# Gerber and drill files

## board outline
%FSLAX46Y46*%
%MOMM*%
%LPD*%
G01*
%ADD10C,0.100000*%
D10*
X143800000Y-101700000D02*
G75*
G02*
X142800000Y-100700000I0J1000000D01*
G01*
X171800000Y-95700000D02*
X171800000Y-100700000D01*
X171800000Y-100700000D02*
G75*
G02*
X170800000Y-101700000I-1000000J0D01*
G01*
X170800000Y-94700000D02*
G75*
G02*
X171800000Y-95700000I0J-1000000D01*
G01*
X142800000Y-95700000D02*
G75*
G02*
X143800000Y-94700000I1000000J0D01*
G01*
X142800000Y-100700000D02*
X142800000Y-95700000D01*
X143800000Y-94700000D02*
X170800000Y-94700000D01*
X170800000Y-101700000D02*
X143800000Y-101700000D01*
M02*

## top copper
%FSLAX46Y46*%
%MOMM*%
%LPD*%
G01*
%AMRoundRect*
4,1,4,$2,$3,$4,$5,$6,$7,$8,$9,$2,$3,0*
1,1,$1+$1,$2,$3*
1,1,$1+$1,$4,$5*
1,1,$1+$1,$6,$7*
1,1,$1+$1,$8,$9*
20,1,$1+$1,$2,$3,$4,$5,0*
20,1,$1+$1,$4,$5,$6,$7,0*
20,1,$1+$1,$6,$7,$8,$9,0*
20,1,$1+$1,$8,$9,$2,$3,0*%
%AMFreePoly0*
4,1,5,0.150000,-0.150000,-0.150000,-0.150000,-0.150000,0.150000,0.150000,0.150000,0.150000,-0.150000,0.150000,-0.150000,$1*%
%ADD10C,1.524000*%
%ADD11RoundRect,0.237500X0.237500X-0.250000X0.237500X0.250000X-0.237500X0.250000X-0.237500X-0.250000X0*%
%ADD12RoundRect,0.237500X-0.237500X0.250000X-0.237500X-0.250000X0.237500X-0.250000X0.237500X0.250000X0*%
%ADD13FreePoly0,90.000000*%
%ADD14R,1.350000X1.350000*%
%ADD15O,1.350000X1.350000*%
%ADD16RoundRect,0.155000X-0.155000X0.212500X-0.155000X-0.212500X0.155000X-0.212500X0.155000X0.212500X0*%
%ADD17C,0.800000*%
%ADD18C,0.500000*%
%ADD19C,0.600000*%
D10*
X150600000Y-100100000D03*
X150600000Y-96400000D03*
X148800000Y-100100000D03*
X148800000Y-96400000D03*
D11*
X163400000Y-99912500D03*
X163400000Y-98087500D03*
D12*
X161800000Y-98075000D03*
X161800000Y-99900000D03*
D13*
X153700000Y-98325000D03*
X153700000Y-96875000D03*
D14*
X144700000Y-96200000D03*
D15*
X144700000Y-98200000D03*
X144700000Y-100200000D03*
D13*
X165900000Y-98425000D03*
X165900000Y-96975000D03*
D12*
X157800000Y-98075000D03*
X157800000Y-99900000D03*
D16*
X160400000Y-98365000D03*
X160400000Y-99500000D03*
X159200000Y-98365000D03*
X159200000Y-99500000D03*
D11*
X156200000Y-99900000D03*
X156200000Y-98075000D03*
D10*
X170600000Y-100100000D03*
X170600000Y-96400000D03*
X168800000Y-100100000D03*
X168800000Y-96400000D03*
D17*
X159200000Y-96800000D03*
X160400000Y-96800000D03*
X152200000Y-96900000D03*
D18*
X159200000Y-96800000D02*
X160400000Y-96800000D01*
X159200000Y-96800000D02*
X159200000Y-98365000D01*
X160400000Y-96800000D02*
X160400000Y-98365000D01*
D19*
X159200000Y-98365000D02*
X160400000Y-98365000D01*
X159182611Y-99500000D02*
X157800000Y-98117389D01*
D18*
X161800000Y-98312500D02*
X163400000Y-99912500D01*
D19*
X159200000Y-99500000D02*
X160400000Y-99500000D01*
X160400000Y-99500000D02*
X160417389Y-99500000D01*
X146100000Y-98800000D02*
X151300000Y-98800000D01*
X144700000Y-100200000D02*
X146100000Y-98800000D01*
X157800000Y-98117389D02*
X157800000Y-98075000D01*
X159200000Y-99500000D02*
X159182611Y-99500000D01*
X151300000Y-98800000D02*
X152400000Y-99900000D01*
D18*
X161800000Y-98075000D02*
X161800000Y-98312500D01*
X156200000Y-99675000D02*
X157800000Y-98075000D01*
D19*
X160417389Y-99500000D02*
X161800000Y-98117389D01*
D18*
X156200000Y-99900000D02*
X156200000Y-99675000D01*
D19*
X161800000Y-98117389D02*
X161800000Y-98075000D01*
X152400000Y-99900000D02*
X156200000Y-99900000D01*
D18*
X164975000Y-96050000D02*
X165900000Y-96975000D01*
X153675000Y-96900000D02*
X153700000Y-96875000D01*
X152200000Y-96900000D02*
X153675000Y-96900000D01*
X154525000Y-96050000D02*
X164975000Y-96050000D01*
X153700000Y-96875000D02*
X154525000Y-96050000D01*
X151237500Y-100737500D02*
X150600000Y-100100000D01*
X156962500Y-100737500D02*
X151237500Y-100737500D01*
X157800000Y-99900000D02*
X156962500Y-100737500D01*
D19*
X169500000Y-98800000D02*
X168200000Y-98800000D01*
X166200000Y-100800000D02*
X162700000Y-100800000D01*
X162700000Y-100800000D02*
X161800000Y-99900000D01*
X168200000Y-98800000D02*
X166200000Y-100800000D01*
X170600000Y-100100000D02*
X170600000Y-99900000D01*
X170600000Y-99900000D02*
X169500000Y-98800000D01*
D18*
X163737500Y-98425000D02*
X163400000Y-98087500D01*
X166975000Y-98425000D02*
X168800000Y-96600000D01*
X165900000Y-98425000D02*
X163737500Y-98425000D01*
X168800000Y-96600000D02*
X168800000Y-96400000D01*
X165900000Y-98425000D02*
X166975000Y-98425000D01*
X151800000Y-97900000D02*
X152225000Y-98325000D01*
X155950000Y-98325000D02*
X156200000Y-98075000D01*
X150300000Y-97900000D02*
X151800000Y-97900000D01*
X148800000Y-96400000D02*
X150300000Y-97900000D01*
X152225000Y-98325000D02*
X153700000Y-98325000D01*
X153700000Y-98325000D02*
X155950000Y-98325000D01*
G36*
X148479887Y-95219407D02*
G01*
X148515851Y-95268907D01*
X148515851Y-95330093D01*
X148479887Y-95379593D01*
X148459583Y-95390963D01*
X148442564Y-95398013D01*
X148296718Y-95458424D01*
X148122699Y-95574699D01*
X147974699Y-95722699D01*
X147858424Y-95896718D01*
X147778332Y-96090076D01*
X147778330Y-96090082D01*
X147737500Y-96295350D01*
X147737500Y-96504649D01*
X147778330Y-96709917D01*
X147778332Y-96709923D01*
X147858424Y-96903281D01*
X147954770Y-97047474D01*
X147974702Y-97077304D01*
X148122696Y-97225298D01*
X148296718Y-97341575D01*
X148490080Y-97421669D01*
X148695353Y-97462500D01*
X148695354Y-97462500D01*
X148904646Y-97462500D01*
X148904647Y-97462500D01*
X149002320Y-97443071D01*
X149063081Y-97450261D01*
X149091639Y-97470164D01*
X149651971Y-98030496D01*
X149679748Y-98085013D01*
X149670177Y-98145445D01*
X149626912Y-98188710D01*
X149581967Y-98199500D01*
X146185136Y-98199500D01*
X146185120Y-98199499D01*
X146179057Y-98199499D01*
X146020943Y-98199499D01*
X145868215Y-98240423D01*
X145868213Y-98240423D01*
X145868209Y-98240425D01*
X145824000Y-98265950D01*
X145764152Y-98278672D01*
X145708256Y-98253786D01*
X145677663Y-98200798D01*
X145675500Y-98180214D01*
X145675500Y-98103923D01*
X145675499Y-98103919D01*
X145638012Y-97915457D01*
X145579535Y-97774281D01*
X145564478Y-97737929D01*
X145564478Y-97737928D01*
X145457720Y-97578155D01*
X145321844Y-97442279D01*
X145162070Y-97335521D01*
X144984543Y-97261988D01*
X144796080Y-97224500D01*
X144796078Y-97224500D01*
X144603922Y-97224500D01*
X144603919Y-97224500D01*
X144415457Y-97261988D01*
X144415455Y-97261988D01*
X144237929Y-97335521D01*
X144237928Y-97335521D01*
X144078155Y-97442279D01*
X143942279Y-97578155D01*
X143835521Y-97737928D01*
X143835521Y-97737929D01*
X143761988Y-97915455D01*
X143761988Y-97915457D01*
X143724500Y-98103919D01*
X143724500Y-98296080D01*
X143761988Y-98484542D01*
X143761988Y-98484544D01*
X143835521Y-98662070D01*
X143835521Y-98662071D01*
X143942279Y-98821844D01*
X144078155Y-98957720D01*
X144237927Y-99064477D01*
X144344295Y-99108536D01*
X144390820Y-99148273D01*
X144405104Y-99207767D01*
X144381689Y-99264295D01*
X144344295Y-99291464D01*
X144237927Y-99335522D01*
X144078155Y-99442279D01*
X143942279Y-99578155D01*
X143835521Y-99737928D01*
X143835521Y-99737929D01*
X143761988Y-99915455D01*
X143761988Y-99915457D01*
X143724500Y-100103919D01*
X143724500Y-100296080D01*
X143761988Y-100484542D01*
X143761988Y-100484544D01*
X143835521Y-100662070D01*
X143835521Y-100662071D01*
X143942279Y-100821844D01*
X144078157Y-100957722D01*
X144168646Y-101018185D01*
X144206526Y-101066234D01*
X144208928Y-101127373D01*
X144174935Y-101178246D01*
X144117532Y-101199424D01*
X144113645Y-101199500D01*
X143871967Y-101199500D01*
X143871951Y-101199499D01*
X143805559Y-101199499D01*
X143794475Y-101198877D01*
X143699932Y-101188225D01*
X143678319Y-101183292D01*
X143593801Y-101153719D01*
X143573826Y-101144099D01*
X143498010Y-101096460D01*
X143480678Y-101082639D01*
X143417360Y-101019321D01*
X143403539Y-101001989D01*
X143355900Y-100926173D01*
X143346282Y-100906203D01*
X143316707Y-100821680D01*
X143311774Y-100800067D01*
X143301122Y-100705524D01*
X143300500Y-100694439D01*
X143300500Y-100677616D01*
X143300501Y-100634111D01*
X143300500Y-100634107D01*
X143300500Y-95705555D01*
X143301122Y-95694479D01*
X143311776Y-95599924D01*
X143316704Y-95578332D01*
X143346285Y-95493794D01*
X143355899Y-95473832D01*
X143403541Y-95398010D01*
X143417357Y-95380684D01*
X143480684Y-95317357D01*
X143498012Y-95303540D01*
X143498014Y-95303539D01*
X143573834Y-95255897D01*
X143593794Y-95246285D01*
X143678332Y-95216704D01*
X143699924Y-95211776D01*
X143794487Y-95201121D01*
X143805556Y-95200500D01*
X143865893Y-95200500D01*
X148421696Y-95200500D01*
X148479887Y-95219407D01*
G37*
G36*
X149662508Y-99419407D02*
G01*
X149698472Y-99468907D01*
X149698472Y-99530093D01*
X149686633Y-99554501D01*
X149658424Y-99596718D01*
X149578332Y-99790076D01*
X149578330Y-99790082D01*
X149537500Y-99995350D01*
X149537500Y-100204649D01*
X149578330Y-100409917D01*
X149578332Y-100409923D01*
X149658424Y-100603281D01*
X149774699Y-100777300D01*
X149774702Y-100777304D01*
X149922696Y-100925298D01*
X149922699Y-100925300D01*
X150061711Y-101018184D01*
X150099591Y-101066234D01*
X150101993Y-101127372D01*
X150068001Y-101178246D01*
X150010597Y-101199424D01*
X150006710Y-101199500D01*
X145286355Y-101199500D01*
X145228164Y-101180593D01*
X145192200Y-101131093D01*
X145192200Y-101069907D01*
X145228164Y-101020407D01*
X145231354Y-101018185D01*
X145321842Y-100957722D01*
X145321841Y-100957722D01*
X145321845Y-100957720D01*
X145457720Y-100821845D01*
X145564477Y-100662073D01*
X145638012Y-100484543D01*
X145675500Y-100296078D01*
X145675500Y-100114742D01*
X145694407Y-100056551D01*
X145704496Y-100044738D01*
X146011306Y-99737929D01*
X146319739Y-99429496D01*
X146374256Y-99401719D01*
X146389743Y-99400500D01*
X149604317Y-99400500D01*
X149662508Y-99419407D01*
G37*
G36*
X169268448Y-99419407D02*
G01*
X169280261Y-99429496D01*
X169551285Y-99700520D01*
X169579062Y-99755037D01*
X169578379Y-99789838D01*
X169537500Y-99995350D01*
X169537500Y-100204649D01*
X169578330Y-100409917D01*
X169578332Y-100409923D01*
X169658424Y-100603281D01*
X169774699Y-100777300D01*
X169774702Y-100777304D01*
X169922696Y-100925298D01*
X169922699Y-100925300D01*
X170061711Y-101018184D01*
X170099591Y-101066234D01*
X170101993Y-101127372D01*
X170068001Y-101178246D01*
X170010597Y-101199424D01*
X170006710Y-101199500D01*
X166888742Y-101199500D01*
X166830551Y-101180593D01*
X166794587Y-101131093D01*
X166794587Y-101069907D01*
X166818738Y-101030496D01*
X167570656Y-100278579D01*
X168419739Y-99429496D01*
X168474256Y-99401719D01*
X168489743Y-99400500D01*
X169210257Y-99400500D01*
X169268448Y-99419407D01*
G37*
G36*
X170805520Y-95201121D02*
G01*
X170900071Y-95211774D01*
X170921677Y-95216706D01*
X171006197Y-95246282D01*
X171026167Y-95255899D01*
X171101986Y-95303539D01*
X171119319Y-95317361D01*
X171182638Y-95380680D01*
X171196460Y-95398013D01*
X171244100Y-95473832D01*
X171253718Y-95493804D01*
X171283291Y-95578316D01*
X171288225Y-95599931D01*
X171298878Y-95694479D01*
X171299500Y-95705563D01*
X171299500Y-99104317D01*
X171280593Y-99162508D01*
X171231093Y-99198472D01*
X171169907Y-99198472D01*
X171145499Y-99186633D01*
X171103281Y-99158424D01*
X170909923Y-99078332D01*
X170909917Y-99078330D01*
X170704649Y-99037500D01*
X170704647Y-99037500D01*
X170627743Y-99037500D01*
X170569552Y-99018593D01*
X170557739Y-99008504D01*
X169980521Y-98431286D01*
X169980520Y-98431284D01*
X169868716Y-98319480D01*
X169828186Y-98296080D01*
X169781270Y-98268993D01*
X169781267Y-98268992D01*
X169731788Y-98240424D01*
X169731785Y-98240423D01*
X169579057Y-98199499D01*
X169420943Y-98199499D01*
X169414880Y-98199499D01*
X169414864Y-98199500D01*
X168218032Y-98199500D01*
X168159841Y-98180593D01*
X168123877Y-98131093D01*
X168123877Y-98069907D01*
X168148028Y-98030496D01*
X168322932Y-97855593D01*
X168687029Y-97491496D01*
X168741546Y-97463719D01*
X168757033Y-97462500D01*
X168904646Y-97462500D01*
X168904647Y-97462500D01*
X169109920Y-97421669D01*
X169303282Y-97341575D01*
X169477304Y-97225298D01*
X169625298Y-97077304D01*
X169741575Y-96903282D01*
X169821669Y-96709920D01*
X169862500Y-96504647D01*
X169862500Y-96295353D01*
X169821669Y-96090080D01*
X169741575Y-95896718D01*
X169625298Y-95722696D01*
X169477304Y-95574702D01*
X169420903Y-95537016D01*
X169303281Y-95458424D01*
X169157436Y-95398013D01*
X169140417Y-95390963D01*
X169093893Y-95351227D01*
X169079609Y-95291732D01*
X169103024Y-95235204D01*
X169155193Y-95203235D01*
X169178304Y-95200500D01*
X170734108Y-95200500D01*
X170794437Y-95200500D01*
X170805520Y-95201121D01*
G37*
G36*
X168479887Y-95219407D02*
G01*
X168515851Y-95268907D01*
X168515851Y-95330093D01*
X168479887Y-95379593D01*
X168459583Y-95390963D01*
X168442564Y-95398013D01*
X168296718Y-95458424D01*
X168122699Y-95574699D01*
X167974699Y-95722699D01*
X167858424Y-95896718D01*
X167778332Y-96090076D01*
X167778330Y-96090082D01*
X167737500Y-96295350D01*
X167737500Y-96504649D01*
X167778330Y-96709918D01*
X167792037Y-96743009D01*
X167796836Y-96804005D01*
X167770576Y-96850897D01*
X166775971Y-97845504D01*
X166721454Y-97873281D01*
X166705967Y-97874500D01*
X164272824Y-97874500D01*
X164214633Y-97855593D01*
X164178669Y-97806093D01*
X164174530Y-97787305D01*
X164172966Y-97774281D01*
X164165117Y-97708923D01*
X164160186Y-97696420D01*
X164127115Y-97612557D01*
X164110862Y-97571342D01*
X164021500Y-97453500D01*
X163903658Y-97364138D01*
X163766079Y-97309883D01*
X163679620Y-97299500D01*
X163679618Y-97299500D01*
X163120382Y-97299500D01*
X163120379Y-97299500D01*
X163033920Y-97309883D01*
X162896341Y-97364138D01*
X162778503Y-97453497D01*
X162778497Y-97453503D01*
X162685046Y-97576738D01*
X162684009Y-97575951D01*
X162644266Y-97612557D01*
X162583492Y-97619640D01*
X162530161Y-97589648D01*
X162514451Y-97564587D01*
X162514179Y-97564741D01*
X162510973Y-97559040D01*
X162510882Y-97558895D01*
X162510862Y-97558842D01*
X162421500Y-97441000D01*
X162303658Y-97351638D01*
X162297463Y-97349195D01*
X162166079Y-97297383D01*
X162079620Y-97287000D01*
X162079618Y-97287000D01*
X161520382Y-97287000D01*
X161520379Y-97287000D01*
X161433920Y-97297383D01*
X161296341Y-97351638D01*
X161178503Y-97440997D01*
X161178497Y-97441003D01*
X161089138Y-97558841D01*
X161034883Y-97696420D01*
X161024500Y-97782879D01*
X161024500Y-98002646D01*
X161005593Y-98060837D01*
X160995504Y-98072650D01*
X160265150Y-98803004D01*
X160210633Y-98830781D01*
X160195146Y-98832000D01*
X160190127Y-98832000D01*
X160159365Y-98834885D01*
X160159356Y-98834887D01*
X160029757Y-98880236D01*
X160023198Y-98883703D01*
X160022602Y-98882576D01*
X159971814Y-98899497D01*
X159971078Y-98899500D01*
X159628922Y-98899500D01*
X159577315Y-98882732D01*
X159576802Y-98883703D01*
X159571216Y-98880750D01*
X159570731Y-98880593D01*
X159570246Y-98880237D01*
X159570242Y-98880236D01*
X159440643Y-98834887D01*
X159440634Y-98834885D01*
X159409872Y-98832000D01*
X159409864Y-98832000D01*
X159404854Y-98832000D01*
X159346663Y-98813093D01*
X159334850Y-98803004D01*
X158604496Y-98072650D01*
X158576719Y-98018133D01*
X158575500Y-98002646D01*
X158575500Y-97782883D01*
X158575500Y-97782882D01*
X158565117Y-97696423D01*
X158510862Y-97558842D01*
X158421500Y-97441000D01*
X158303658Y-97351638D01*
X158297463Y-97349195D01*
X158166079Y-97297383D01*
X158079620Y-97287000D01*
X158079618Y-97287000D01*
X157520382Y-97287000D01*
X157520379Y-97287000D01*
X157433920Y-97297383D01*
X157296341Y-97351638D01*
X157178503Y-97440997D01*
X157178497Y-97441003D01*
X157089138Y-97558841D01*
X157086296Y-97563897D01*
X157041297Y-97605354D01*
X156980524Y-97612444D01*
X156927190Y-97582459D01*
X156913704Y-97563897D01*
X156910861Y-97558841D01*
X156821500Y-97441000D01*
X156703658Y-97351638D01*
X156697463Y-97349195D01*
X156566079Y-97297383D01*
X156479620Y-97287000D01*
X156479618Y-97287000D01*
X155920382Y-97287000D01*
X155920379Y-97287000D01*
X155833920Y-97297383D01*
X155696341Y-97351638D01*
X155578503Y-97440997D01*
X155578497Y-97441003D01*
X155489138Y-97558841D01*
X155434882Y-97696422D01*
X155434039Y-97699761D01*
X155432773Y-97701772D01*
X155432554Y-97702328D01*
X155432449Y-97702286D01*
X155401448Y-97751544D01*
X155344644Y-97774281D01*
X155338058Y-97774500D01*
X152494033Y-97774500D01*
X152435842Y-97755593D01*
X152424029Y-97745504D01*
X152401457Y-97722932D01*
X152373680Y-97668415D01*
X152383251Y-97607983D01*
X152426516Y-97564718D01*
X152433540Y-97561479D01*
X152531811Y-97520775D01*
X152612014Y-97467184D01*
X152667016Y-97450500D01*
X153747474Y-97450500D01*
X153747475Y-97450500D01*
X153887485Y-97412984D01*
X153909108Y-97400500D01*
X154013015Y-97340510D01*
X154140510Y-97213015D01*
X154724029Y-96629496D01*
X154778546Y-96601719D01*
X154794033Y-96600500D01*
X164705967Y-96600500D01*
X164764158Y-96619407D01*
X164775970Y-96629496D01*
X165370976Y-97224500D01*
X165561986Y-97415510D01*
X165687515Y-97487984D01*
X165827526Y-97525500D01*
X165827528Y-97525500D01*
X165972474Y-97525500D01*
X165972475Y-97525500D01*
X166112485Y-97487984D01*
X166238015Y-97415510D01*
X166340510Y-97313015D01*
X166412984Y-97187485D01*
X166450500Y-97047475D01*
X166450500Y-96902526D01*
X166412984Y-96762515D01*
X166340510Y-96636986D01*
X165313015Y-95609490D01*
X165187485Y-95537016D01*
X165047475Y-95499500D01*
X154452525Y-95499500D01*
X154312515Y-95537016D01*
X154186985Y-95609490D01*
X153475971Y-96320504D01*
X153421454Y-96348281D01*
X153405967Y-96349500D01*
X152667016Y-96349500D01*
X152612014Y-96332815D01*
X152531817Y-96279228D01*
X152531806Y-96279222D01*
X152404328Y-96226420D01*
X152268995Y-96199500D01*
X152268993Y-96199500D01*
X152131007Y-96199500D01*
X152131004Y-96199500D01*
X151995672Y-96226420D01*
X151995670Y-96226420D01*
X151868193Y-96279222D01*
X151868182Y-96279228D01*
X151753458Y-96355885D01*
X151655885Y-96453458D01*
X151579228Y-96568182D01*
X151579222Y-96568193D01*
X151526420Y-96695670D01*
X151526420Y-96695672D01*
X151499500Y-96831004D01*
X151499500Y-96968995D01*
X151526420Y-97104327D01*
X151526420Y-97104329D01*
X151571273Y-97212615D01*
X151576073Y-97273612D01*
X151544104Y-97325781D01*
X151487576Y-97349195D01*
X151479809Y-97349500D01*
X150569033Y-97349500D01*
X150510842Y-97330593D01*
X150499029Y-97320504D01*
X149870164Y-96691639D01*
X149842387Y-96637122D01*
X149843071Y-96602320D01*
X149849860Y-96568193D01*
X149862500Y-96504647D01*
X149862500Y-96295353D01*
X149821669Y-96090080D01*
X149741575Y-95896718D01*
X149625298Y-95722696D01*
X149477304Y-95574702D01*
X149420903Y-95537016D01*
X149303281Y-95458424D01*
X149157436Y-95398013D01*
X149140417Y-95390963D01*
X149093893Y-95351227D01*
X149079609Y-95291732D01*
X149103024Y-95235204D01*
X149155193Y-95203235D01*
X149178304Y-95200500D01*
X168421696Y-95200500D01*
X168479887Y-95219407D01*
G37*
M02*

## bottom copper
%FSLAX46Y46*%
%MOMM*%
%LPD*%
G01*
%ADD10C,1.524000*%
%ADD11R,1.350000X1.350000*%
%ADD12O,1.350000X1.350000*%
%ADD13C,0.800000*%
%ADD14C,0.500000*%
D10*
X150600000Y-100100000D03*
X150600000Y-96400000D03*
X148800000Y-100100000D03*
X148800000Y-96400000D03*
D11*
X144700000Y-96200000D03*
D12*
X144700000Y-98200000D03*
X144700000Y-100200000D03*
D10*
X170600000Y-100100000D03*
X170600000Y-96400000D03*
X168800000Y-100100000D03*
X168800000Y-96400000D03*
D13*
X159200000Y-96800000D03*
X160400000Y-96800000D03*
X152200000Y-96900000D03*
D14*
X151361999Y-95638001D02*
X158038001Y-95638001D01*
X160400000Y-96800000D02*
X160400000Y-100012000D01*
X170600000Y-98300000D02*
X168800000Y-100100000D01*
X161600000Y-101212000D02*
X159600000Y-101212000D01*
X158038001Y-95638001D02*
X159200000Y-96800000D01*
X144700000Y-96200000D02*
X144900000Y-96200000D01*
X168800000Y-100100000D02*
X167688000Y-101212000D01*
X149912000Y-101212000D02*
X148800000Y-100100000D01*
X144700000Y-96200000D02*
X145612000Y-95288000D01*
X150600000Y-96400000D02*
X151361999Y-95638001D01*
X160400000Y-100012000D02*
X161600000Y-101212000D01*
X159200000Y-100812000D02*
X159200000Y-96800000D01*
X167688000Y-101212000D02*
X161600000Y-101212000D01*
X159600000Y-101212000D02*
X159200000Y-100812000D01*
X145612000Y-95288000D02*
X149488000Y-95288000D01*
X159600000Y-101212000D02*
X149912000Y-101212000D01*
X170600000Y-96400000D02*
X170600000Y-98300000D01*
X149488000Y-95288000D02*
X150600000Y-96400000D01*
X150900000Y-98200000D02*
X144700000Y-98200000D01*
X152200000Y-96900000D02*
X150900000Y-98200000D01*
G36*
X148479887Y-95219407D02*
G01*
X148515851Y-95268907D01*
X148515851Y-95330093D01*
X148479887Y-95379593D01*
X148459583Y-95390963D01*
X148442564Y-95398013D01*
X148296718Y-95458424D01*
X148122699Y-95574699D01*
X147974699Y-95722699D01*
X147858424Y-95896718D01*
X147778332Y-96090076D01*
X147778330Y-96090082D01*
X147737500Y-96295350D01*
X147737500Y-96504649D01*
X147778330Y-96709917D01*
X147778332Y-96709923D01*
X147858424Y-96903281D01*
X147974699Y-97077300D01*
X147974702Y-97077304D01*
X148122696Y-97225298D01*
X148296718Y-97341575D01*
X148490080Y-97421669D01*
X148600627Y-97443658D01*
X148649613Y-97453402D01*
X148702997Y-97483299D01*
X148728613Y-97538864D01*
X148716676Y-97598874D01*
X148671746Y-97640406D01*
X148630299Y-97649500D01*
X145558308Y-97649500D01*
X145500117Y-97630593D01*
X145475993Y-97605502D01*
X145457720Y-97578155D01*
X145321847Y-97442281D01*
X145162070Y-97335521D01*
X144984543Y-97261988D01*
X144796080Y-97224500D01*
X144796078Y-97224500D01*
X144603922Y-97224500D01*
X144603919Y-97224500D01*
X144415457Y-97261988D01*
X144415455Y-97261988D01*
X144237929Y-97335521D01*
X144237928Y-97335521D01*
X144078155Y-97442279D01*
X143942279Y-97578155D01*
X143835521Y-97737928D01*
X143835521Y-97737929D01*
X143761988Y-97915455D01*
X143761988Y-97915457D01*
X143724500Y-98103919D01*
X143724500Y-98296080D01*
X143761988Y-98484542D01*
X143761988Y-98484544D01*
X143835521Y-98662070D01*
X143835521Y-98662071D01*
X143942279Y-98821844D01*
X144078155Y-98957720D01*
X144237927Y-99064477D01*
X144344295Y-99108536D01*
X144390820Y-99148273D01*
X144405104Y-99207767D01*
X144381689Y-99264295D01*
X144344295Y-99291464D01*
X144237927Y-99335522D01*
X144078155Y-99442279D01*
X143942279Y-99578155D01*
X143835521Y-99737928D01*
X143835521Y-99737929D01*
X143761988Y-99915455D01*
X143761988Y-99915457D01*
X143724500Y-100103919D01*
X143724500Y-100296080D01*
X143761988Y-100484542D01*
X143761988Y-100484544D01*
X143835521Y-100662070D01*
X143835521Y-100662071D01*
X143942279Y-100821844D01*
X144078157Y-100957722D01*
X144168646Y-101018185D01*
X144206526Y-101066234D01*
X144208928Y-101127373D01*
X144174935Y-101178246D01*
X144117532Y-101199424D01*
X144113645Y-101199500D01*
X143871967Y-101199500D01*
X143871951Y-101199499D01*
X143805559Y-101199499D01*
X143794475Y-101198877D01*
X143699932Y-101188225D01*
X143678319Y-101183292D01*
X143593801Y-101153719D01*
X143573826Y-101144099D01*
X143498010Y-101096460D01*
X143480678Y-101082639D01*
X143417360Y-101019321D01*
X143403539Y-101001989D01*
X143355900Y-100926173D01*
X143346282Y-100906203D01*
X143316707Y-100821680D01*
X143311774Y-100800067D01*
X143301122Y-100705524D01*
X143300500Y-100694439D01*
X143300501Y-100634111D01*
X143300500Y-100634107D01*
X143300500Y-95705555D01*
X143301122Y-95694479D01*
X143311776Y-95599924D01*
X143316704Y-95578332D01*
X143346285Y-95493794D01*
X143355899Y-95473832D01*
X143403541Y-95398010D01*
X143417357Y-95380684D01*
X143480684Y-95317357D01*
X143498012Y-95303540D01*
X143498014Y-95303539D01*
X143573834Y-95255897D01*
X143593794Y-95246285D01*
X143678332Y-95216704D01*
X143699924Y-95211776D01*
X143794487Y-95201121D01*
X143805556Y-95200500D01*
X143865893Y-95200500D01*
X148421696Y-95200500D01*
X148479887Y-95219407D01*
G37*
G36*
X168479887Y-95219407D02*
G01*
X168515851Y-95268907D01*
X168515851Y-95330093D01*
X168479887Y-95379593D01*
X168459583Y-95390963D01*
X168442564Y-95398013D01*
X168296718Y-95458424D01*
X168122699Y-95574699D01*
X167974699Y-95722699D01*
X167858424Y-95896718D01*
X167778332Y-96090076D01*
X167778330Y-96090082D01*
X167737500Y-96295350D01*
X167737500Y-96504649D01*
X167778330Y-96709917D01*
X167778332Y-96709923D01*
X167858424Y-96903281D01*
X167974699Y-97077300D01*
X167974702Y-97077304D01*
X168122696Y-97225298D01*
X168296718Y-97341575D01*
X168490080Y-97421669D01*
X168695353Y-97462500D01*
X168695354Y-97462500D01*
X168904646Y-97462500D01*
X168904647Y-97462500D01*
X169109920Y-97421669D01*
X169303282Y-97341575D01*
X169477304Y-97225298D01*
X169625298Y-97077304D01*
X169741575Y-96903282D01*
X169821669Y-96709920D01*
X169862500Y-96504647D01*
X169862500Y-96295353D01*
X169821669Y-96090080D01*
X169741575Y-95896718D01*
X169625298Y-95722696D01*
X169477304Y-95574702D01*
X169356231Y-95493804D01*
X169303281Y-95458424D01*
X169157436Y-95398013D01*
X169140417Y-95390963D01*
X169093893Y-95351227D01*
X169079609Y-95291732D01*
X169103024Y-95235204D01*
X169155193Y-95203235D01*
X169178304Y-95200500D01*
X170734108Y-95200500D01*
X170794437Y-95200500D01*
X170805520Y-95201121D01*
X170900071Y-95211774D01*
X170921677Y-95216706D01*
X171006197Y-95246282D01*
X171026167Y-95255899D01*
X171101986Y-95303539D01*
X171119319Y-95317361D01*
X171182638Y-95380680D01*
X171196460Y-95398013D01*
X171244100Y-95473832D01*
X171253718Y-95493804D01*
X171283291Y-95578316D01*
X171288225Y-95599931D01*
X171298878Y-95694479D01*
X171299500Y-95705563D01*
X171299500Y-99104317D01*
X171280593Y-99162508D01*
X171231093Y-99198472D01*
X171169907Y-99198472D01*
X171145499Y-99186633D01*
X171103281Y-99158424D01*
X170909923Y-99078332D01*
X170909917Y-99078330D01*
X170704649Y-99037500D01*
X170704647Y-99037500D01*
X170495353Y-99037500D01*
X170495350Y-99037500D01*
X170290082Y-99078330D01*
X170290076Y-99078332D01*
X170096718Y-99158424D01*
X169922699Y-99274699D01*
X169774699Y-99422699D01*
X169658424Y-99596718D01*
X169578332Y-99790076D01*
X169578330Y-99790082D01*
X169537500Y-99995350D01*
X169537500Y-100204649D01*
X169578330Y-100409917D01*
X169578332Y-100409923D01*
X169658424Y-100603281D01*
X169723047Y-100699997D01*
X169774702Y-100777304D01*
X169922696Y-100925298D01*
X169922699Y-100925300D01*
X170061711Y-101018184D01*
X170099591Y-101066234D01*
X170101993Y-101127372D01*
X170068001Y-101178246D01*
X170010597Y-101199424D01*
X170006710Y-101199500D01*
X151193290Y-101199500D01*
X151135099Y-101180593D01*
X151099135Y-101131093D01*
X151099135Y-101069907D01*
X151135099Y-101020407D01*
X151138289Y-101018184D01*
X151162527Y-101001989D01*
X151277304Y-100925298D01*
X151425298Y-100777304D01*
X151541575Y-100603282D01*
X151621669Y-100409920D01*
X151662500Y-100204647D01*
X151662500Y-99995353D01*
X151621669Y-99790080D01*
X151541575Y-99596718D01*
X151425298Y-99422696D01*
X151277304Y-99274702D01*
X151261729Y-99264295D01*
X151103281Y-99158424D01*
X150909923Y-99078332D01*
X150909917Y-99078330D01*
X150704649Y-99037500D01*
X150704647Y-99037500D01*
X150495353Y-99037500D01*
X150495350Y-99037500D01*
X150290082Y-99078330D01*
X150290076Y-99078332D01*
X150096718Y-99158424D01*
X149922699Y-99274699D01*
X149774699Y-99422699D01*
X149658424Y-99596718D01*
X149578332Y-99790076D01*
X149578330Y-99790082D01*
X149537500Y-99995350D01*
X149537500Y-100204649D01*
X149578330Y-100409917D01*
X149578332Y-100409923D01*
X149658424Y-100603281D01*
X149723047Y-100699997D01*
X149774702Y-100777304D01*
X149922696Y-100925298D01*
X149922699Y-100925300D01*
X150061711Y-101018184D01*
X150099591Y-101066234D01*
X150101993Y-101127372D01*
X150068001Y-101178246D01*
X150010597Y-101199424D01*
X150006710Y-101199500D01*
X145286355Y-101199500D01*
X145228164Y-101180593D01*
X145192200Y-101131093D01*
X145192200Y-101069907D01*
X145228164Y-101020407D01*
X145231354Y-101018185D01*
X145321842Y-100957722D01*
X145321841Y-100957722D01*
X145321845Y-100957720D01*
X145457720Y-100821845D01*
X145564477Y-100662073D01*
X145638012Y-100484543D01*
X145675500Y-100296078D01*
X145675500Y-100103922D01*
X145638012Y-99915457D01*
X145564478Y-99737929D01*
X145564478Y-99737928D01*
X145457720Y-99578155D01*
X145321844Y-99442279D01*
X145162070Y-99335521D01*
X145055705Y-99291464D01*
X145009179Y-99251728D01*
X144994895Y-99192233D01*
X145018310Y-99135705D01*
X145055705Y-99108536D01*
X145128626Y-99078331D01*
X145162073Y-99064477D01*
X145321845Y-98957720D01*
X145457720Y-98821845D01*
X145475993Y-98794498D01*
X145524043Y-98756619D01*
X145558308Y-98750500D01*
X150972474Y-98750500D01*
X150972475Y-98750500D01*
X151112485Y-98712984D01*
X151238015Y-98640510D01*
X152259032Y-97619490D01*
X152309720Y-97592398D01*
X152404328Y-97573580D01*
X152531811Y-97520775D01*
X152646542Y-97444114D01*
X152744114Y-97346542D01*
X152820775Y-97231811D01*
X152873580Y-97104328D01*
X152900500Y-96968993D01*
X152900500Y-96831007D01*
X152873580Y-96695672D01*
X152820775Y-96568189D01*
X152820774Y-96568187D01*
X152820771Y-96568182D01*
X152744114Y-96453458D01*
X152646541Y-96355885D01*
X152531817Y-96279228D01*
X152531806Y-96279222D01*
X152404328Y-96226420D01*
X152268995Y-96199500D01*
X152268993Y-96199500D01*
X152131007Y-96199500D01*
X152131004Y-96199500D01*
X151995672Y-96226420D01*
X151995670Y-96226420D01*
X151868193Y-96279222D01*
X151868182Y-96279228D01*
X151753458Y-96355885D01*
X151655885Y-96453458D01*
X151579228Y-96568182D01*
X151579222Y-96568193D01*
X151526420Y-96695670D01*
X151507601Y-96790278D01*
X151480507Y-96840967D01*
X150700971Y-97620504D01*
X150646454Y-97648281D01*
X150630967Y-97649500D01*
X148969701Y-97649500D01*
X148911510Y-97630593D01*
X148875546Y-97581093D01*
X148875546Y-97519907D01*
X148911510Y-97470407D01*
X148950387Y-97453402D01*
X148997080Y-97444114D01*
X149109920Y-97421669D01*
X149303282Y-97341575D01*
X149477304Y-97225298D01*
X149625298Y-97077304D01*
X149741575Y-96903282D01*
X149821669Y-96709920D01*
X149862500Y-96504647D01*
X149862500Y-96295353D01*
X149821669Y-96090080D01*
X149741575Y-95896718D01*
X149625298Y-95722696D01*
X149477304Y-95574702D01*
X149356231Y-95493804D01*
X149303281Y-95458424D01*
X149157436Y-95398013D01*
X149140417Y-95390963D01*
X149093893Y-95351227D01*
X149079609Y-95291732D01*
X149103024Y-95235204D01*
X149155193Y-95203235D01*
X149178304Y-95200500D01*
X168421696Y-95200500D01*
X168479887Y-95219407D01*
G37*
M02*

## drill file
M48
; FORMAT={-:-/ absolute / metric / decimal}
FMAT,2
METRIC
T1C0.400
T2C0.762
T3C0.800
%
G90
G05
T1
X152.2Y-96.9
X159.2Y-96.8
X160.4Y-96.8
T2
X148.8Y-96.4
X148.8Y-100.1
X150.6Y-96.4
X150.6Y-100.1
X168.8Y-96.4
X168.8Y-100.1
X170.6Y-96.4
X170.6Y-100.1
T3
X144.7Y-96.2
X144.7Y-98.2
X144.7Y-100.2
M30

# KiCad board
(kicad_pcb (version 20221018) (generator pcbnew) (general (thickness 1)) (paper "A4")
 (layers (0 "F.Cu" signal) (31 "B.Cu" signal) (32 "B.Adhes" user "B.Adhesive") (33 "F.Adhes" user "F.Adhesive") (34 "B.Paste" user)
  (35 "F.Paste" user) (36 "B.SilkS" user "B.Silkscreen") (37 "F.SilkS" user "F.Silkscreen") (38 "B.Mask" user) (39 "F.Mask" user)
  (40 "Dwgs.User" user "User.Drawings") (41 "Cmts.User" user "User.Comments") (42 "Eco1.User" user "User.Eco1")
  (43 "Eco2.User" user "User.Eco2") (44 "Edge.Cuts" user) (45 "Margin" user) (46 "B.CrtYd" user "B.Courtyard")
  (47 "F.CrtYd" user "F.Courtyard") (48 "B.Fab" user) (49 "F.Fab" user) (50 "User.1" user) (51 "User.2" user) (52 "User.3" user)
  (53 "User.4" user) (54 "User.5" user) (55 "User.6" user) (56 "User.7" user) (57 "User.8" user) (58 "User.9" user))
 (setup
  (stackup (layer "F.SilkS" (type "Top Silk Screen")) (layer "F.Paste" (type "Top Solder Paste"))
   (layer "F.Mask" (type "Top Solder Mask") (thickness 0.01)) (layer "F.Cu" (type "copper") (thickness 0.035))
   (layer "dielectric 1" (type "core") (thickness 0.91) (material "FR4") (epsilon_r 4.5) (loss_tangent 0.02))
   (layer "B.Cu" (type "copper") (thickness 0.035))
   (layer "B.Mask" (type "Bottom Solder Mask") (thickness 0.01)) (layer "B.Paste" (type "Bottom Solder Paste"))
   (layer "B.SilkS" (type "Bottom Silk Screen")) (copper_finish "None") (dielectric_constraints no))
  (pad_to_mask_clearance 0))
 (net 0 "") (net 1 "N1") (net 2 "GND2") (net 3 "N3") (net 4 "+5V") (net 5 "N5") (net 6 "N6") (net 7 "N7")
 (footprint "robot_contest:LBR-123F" (layer "F.Cu") (at 149.7 98.25 90)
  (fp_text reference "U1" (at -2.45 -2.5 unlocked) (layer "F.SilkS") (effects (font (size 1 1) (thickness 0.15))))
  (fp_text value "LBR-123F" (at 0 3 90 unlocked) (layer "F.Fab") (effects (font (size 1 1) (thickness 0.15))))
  (pad "1" thru_hole circle (at -1.85 0.9 90) (size 1.524 1.524) (drill 0.762) (layers "*.Cu" "*.Mask") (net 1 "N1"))
  (pad "2" thru_hole circle (at 1.85 0.9 90) (size 1.524 1.524) (drill 0.762) (layers "*.Cu" "*.Mask") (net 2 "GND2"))
  (pad "3" thru_hole circle (at -1.85 -0.9 90) (size 1.524 1.524) (drill 0.762) (layers "*.Cu" "*.Mask") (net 2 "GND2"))
  (pad "4" thru_hole circle (at 1.85 -0.9 90) (size 1.524 1.524) (drill 0.762) (layers "*.Cu" "*.Mask") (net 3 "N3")))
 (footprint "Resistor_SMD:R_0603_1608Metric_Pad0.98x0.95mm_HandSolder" (layer "F.Cu") (at 163.4 99 90)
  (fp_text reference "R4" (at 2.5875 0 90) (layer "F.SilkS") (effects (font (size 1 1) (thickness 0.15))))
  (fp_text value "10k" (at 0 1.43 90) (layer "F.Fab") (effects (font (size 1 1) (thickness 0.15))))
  (pad "1" smd roundrect (at -0.9125 0 90) (size 0.975 0.95) (layers "F.Cu" "F.Paste" "F.Mask") (roundrect_rratio 0.25) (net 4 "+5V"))
  (pad "2" smd roundrect (at 0.9125 0 90) (size 0.975 0.95) (layers "F.Cu" "F.Paste" "F.Mask") (roundrect_rratio 0.25) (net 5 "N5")))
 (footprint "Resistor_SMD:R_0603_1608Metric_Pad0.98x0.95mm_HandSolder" (layer "F.Cu") (at 161.8 98.9875 -90)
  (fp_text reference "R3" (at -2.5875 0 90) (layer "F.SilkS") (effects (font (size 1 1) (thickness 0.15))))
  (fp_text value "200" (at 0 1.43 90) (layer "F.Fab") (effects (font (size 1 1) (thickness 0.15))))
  (pad "1" smd roundrect (at -0.9125 0 270) (size 0.975 0.95) (layers "F.Cu" "F.Paste" "F.Mask") (roundrect_rratio 0.25) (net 4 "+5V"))
  (pad "2" smd roundrect (at 0.9125 0 270) (size 0.975 0.95) (layers "F.Cu" "F.Paste" "F.Mask") (roundrect_rratio 0.25) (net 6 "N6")))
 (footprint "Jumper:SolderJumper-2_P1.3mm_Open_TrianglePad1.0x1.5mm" (layer "F.Cu") (at 153.7 97.6 90)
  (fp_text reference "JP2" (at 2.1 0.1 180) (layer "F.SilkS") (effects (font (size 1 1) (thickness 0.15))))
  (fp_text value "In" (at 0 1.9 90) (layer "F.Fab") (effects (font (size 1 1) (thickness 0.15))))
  (pad "1" smd custom (at -0.725 0 90) (size 0.3 0.3) (layers "F.Cu" "F.Mask") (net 3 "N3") (zone_connect 2) (thermal_bridge_angle 45)
   (options (clearance outline) (anchor rect)) (primitives))
  (pad "2" smd custom (at 0.725 0 90) (size 0.3 0.3) (layers "F.Cu" "F.Mask") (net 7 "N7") (zone_connect 2) (thermal_bridge_angle 45)
   (options (clearance outline) (anchor rect)) (primitives)))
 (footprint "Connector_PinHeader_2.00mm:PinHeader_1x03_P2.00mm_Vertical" (layer "F.Cu") (at 144.7 96.2)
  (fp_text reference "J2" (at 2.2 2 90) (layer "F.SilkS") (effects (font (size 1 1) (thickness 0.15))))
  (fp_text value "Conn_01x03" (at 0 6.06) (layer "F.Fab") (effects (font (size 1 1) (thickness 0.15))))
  (pad "1" thru_hole rect (at 0 0) (size 1.35 1.35) (drill 0.8) (layers "*.Cu" "*.Mask") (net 2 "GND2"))
  (pad "2" thru_hole oval (at 0 2) (size 1.35 1.35) (drill 0.8) (layers "*.Cu" "*.Mask") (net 7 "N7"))
  (pad "3" thru_hole oval (at 0 4) (size 1.35 1.35) (drill 0.8) (layers "*.Cu" "*.Mask") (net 4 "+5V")))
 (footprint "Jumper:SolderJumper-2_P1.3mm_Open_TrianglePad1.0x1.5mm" (layer "F.Cu") (at 165.9 97.7 90)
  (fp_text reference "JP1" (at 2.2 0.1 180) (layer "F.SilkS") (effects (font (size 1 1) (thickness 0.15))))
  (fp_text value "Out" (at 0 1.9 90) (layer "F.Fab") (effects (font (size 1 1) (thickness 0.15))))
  (pad "1" smd custom (at -0.725 0 90) (size 0.3 0.3) (layers "F.Cu" "F.Mask") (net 5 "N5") (zone_connect 2) (thermal_bridge_angle 45)
   (options (clearance outline) (anchor rect)) (primitives))
  (pad "2" smd custom (at 0.725 0 90) (size 0.3 0.3) (layers "F.Cu" "F.Mask") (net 7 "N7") (zone_connect 2) (thermal_bridge_angle 45)
   (options (clearance outline) (anchor rect)) (primitives)))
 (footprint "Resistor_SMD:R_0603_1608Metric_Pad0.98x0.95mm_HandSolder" (layer "F.Cu") (at 157.8 98.9875 -90)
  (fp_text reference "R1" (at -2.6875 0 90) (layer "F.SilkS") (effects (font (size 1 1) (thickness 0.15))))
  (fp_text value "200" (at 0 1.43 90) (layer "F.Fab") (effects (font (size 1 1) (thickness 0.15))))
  (pad "1" smd roundrect (at -0.9125 0 270) (size 0.975 0.95) (layers "F.Cu" "F.Paste" "F.Mask") (roundrect_rratio 0.25) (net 4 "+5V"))
  (pad "2" smd roundrect (at 0.9125 0 270) (size 0.975 0.95) (layers "F.Cu" "F.Paste" "F.Mask") (roundrect_rratio 0.25) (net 1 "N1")))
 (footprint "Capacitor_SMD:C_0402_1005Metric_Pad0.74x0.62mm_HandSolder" (layer "F.Cu") (at 160.4 98.9325 -90)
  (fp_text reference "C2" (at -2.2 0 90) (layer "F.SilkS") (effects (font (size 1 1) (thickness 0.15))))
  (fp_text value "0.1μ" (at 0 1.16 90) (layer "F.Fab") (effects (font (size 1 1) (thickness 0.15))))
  (pad "1" smd roundrect (at -0.5675 0 270) (size 0.735 0.62) (layers "F.Cu" "F.Paste" "F.Mask") (roundrect_rratio 0.25) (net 2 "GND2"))
  (pad "2" smd roundrect (at 0.5675 0 270) (size 0.735 0.62) (layers "F.Cu" "F.Paste" "F.Mask") (roundrect_rratio 0.25) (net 4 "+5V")))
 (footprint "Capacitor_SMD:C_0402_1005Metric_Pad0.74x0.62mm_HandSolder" (layer "F.Cu") (at 159.2 98.9325 -90)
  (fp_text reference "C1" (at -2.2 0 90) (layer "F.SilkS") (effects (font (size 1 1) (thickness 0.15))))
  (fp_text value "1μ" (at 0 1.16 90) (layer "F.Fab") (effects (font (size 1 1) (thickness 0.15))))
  (pad "1" smd roundrect (at -0.5675 0 270) (size 0.735 0.62) (layers "F.Cu" "F.Paste" "F.Mask") (roundrect_rratio 0.25) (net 2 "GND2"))
  (pad "2" smd roundrect (at 0.5675 0 270) (size 0.735 0.62) (layers "F.Cu" "F.Paste" "F.Mask") (roundrect_rratio 0.25) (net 4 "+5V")))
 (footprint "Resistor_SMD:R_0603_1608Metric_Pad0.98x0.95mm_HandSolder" (layer "F.Cu") (at 156.2 98.9875 90)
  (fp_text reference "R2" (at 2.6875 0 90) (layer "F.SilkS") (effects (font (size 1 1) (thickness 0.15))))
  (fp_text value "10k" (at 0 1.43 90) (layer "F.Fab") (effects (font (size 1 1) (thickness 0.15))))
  (pad "1" smd roundrect (at -0.9125 0 90) (size 0.975 0.95) (layers "F.Cu" "F.Paste" "F.Mask") (roundrect_rratio 0.25) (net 4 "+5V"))
  (pad "2" smd roundrect (at 0.9125 0 90) (size 0.975 0.95) (layers "F.Cu" "F.Paste" "F.Mask") (roundrect_rratio 0.25) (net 3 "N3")))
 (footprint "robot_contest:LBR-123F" (layer "F.Cu") (at 169.7 98.25 90)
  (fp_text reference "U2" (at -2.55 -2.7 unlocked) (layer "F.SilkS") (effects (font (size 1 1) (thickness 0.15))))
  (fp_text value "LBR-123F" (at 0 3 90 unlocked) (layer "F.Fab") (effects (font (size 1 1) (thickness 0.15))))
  (pad "1" thru_hole circle (at -1.85 0.9 90) (size 1.524 1.524) (drill 0.762) (layers "*.Cu" "*.Mask") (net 6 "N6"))
  (pad "2" thru_hole circle (at 1.85 0.9 90) (size 1.524 1.524) (drill 0.762) (layers "*.Cu" "*.Mask") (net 2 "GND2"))
  (pad "3" thru_hole circle (at -1.85 -0.9 90) (size 1.524 1.524) (drill 0.762) (layers "*.Cu" "*.Mask") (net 2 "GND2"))
  (pad "4" thru_hole circle (at 1.85 -0.9 90) (size 1.524 1.524) (drill 0.762) (layers "*.Cu" "*.Mask") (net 5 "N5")))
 (gr_arc (start 143.8 101.7) (mid 143.092892 101.407109) (end 142.8 100.7) (stroke (width 0.1) (type default)) (layer "Edge.Cuts"))
 (gr_line (start 171.8 95.7) (end 171.8 100.7) (stroke (width 0.1) (type default)) (layer "Edge.Cuts"))
 (gr_arc (start 171.8 100.7) (mid 171.507107 101.407107) (end 170.8 101.7) (stroke (width 0.1) (type default)) (layer "Edge.Cuts"))
 (gr_arc (start 170.8 94.7) (mid 171.507107 94.992893) (end 171.8 95.7) (stroke (width 0.1) (type default)) (layer "Edge.Cuts"))
 (gr_arc (start 142.8 95.7) (mid 143.092893 94.992894) (end 143.8 94.7) (stroke (width 0.1) (type default)) (layer "Edge.Cuts"))
 (gr_line (start 142.8 100.7) (end 142.8 95.7) (stroke (width 0.1) (type default)) (layer "Edge.Cuts"))
 (gr_line (start 143.8 94.7) (end 170.8 94.7) (stroke (width 0.1) (type default)) (layer "Edge.Cuts"))
 (gr_line (start 170.8 101.7) (end 143.8 101.7) (stroke (width 0.1) (type default)) (layer "Edge.Cuts"))
 (segment (start 159.2 96.8) (end 160.4 96.8) (width 0.5) (layer "F.Cu") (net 2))
 (segment (start 159.2 96.8) (end 159.2 98.365) (width 0.5) (layer "F.Cu") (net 2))
 (segment (start 160.4 96.8) (end 160.4 98.365) (width 0.5) (layer "F.Cu") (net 2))
 (segment (start 159.2 98.365) (end 160.4 98.365) (width 0.6) (layer "F.Cu") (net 2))
 (via (at 159.2 96.8) (size 0.8) (drill 0.4) (layers "F.Cu" "B.Cu") (free) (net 2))
 (via (at 160.4 96.8) (size 0.8) (drill 0.4) (layers "F.Cu" "B.Cu") (free) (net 2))
 (segment (start 151.361999 95.638001) (end 158.038001 95.638001) (width 0.5) (layer "B.Cu") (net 2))
 (segment (start 160.4 96.8) (end 160.4 100.012) (width 0.5) (layer "B.Cu") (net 2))
 (segment (start 170.6 98.3) (end 168.8 100.1) (width 0.5) (layer "B.Cu") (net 2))
 (segment (start 161.6 101.212) (end 159.6 101.212) (width 0.5) (layer "B.Cu") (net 2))
 (segment (start 158.038001 95.638001) (end 159.2 96.8) (width 0.5) (layer "B.Cu") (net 2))
 (segment (start 144.7 96.2) (end 144.9 96.2) (width 0.5) (layer "B.Cu") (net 2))
 (segment (start 168.8 100.1) (end 167.688 101.212) (width 0.5) (layer "B.Cu") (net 2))
 (segment (start 149.912 101.212) (end 148.8 100.1) (width 0.5) (layer "B.Cu") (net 2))
 (segment (start 144.7 96.2) (end 145.612 95.288) (width 0.5) (layer "B.Cu") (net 2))
 (segment (start 150.6 96.4) (end 151.361999 95.638001) (width 0.5) (layer "B.Cu") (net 2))
 (segment (start 160.4 100.012) (end 161.6 101.212) (width 0.5) (layer "B.Cu") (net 2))
 (segment (start 159.2 100.812) (end 159.2 96.8) (width 0.5) (layer "B.Cu") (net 2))
 (segment (start 167.688 101.212) (end 161.6 101.212) (width 0.5) (layer "B.Cu") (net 2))
 (segment (start 159.6 101.212) (end 159.2 100.812) (width 0.5) (layer "B.Cu") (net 2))
 (segment (start 145.612 95.288) (end 149.488 95.288) (width 0.5) (layer "B.Cu") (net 2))
 (segment (start 159.6 101.212) (end 149.912 101.212) (width 0.5) (layer "B.Cu") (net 2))
 (segment (start 170.6 96.4) (end 170.6 98.3) (width 0.5) (layer "B.Cu") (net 2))
 (segment (start 149.488 95.288) (end 150.6 96.4) (width 0.5) (layer "B.Cu") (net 2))
 (segment (start 159.182611 99.5) (end 157.8 98.117389) (width 0.6) (layer "F.Cu") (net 4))
 (segment (start 161.8 98.3125) (end 163.4 99.9125) (width 0.5) (layer "F.Cu") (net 4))
 (segment (start 159.2 99.5) (end 160.4 99.5) (width 0.6) (layer "F.Cu") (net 4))
 (segment (start 160.4 99.5) (end 160.417389 99.5) (width 0.6) (layer "F.Cu") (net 4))
 (segment (start 146.1 98.8) (end 151.3 98.8) (width 0.6) (layer "F.Cu") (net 4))
 (segment (start 144.7 100.2) (end 146.1 98.8) (width 0.6) (layer "F.Cu") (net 4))
 (segment (start 157.8 98.117389) (end 157.8 98.075) (width 0.6) (layer "F.Cu") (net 4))
 (segment (start 159.2 99.5) (end 159.182611 99.5) (width 0.6) (layer "F.Cu") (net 4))
 (segment (start 151.3 98.8) (end 152.4 99.9) (width 0.6) (layer "F.Cu") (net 4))
 (segment (start 161.8 98.075) (end 161.8 98.3125) (width 0.5) (layer "F.Cu") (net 4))
 (segment (start 156.2 99.675) (end 157.8 98.075) (width 0.5) (layer "F.Cu") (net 4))
 (segment (start 160.417389 99.5) (end 161.8 98.117389) (width 0.6) (layer "F.Cu") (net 4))
 (segment (start 156.2 99.9) (end 156.2 99.675) (width 0.5) (layer "F.Cu") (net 4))
 (segment (start 161.8 98.117389) (end 161.8 98.075) (width 0.6) (layer "F.Cu") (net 4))
 (segment (start 152.4 99.9) (end 156.2 99.9) (width 0.6) (layer "F.Cu") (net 4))
 (segment (start 164.975 96.05) (end 165.9 96.975) (width 0.5) (layer "F.Cu") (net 7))
 (segment (start 153.675 96.9) (end 153.7 96.875) (width 0.5) (layer "F.Cu") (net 7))
 (segment (start 152.2 96.9) (end 153.675 96.9) (width 0.5) (layer "F.Cu") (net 7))
 (segment (start 154.525 96.05) (end 164.975 96.05) (width 0.5) (layer "F.Cu") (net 7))
 (segment (start 153.7 96.875) (end 154.525 96.05) (width 0.5) (layer "F.Cu") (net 7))
 (via (at 152.2 96.9) (size 0.8) (drill 0.4) (layers "F.Cu" "B.Cu") (free) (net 7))
 (segment (start 150.9 98.2) (end 144.7 98.2) (width 0.5) (layer "B.Cu") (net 7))
 (segment (start 152.2 96.9) (end 150.9 98.2) (width 0.5) (layer "B.Cu") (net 7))
 (segment (start 151.2375 100.7375) (end 150.6 100.1) (width 0.5) (layer "F.Cu") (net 1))
 (segment (start 156.9625 100.7375) (end 151.2375 100.7375) (width 0.5) (layer "F.Cu") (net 1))
 (segment (start 157.8 99.9) (end 156.9625 100.7375) (width 0.5) (layer "F.Cu") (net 1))
 (segment (start 169.5 98.8) (end 168.2 98.8) (width 0.6) (layer "F.Cu") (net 6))
 (segment (start 166.2 100.8) (end 162.7 100.8) (width 0.6) (layer "F.Cu") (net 6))
 (segment (start 162.7 100.8) (end 161.8 99.9) (width 0.6) (layer "F.Cu") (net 6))
 (segment (start 168.2 98.8) (end 166.2 100.8) (width 0.6) (layer "F.Cu") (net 6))
 (segment (start 170.6 100.1) (end 170.6 99.9) (width 0.6) (layer "F.Cu") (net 6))
 (segment (start 170.6 99.9) (end 169.5 98.8) (width 0.6) (layer "F.Cu") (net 6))
 (segment (start 163.7375 98.425) (end 163.4 98.0875) (width 0.5) (layer "F.Cu") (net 5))
 (segment (start 166.975 98.425) (end 168.8 96.6) (width 0.5) (layer "F.Cu") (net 5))
 (segment (start 165.9 98.425) (end 163.7375 98.425) (width 0.5) (layer "F.Cu") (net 5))
 (segment (start 168.8 96.6) (end 168.8 96.4) (width 0.5) (layer "F.Cu") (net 5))
 (segment (start 165.9 98.425) (end 166.975 98.425) (width 0.5) (layer "F.Cu") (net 5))
 (segment (start 151.8 97.9) (end 152.225 98.325) (width 0.5) (layer "F.Cu") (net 3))
 (segment (start 155.95 98.325) (end 156.2 98.075) (width 0.5) (layer "F.Cu") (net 3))
 (segment (start 150.3 97.9) (end 151.8 97.9) (width 0.5) (layer "F.Cu") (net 3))
 (segment (start 148.8 96.4) (end 150.3 97.9) (width 0.5) (layer "F.Cu") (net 3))
 (segment (start 152.225 98.325) (end 153.7 98.325) (width 0.5) (layer "F.Cu") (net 3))
 (segment (start 153.7 98.325) (end 155.95 98.325) (width 0.5) (layer "F.Cu") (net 3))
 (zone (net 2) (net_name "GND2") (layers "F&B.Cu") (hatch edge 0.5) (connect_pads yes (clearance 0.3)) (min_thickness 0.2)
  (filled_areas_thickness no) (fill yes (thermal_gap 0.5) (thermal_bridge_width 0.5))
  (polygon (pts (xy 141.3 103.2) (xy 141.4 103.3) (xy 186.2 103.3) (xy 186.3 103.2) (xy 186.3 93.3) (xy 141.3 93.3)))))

